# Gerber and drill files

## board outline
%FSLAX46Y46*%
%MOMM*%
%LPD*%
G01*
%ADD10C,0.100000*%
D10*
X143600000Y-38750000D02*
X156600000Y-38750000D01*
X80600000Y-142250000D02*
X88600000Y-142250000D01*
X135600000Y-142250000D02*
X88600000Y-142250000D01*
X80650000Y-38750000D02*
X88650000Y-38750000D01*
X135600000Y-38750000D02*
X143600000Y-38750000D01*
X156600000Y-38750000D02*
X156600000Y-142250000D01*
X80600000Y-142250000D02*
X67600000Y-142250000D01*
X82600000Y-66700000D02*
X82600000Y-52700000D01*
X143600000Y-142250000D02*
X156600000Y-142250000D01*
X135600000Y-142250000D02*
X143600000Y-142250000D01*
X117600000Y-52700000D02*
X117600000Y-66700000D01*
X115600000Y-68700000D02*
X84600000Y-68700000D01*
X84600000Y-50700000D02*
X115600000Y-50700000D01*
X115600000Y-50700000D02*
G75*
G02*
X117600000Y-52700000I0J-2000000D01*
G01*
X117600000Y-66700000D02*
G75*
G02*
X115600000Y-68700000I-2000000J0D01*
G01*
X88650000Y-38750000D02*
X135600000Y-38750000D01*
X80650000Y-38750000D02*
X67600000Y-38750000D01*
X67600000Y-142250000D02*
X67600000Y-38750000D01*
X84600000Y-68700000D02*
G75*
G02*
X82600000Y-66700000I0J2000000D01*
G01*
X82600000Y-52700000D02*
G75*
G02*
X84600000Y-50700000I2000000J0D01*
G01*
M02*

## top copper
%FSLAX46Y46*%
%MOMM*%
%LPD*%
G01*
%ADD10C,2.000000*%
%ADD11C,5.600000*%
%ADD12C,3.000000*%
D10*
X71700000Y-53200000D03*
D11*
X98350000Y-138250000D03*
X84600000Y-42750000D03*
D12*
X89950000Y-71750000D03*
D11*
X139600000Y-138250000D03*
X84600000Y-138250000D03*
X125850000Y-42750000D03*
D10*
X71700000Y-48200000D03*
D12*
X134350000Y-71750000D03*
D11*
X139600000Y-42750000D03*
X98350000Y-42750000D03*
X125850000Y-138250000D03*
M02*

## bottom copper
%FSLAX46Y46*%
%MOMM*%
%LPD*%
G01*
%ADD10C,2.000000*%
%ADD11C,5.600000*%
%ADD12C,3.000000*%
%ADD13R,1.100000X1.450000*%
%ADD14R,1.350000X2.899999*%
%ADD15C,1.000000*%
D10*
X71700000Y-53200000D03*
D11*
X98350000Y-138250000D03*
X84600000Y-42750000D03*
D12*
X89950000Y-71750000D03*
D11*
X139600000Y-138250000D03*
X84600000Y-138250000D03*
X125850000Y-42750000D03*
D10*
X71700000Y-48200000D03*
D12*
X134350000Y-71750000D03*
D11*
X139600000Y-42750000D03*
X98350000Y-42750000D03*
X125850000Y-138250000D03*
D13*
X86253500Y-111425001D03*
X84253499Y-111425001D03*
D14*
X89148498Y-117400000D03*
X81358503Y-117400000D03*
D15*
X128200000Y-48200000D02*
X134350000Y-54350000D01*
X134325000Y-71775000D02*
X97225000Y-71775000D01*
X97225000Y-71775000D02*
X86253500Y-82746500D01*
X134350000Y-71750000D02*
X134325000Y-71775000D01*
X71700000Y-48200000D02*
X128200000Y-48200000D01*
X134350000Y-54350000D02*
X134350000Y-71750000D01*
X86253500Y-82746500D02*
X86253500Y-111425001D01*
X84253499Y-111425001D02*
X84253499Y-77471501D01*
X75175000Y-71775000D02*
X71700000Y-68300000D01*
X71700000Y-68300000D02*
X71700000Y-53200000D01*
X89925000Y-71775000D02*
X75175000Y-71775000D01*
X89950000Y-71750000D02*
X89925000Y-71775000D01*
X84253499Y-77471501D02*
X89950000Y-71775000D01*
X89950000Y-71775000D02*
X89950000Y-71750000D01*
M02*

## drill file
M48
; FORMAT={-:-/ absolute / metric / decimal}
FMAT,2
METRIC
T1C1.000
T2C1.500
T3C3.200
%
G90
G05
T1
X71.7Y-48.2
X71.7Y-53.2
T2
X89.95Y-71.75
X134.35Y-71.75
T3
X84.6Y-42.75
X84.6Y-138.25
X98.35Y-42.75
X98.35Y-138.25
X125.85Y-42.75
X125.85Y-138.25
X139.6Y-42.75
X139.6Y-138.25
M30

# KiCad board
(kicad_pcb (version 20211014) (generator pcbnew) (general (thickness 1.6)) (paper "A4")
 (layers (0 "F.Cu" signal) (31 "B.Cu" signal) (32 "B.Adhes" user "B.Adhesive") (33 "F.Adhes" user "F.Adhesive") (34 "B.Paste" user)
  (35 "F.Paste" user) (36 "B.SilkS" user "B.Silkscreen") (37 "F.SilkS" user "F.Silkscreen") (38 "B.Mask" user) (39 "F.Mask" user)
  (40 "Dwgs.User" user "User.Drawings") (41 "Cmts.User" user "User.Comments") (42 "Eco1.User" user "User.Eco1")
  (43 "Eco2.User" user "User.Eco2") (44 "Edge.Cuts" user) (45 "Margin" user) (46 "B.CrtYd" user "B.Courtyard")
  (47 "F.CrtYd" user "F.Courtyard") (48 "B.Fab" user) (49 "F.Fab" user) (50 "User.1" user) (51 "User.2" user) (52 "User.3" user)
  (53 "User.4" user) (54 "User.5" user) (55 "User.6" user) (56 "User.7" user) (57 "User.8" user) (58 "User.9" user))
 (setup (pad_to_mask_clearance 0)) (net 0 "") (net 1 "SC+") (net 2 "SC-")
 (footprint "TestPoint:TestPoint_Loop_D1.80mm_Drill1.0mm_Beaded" (layer "F.Cu") (at 71.75 53.2)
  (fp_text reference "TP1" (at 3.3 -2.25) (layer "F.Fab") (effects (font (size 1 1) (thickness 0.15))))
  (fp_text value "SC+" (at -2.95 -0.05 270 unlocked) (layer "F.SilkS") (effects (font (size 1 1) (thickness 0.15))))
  (pad "1" thru_hole circle (at -0.05 0) (size 2 2) (drill 1) (layers *.Cu *.Mask) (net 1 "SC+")))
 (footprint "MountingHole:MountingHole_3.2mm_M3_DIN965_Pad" (layer "F.Cu") (at 98.35 138.25)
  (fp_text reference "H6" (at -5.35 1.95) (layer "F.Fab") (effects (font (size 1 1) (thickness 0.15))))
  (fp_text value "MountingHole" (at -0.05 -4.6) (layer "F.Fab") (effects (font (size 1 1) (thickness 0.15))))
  (pad "1" thru_hole circle (at 0 0) (size 5.6 5.6) (drill 3.2) (layers *.Cu *.Mask)))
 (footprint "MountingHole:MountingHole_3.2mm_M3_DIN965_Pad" (layer "F.Cu") (at 84.6 42.75)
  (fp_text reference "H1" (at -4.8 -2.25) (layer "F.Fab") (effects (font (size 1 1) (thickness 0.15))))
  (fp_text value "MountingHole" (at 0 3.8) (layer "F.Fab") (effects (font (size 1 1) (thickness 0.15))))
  (pad "1" thru_hole circle (at 0 0) (size 5.6 5.6) (drill 3.2) (layers *.Cu *.Mask)))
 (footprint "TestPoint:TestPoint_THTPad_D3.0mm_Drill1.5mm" (layer "F.Cu") (at 89.95 71.75)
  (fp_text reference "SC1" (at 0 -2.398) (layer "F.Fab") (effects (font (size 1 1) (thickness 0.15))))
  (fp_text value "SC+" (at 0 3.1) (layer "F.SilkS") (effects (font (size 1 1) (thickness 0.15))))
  (pad "1" thru_hole circle (at 0 0) (size 3 3) (drill 1.5) (layers *.Cu *.Mask) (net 1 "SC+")))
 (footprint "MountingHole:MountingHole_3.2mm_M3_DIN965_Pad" (layer "F.Cu") (at 139.6 138.25)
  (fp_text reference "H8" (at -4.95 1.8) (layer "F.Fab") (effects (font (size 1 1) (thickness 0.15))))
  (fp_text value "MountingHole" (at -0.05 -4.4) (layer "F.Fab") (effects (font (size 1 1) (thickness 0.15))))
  (pad "1" thru_hole circle (at 0 0) (size 5.6 5.6) (drill 3.2) (layers *.Cu *.Mask)))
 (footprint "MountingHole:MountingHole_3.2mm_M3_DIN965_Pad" (layer "F.Cu") (at 84.6 138.25)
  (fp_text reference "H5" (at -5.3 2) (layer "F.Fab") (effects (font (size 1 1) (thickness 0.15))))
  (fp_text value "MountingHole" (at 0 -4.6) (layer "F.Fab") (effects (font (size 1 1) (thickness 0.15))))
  (pad "1" thru_hole circle (at 0 0) (size 5.6 5.6) (drill 3.2) (layers *.Cu *.Mask)))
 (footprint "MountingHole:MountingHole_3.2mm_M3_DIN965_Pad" (layer "F.Cu") (at 125.85 42.75)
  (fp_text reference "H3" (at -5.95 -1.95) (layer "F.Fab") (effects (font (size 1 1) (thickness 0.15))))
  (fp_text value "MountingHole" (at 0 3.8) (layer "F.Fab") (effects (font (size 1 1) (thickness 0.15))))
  (pad "1" thru_hole circle (at 0 0) (size 5.6 5.6) (drill 3.2) (layers *.Cu *.Mask)))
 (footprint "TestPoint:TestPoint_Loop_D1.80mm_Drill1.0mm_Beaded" (layer "F.Cu") (at 71.7 48.3)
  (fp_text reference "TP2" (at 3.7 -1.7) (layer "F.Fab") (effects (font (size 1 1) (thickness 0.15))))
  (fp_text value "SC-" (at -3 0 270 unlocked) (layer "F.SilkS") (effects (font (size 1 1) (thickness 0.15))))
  (pad "1" thru_hole circle (at 0 -0.1) (size 2 2) (drill 1) (layers *.Cu *.Mask) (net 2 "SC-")))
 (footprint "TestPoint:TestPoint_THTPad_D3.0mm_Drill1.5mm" (layer "F.Cu") (at 134.35 71.75)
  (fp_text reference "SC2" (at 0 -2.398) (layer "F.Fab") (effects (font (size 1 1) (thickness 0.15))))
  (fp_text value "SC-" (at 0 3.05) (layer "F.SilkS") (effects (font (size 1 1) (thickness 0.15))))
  (pad "1" thru_hole circle (at 0 0) (size 3 3) (drill 1.5) (layers *.Cu *.Mask) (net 2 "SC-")))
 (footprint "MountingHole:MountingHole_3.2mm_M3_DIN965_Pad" (layer "F.Cu") (at 139.6 42.75)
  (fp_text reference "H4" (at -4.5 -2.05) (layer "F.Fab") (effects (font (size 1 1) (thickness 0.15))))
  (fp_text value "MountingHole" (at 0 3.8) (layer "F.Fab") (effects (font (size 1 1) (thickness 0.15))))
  (pad "1" thru_hole circle (at 0 0) (size 5.6 5.6) (drill 3.2) (layers *.Cu *.Mask)))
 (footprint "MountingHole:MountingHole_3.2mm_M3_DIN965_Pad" (layer "F.Cu") (at 98.35 42.75)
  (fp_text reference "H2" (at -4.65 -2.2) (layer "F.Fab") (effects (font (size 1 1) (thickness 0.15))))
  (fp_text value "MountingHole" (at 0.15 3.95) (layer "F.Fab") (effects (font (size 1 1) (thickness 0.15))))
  (pad "1" thru_hole circle (at 0 0) (size 5.6 5.6) (drill 3.2) (layers *.Cu *.Mask)))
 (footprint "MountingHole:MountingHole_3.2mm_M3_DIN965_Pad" (layer "F.Cu") (at 125.85 138.25)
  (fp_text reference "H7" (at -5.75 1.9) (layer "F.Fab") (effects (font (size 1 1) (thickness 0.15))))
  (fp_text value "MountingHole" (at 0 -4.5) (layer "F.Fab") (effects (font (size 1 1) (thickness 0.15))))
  (pad "1" thru_hole circle (at 0 0) (size 5.6 5.6) (drill 3.2) (layers *.Cu *.Mask)))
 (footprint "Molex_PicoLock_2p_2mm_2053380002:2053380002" (layer "B.Cu") (at 86.2535 111.425001)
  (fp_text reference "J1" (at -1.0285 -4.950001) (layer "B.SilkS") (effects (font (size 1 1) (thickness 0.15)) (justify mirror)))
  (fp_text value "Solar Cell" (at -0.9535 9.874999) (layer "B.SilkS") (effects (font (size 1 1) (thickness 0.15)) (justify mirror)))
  (pad "1" smd rect locked (at 0 0) (size 1.1 1.45) (layers "B.Cu" "B.Paste" "B.Mask") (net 2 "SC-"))
  (pad "2" smd rect locked (at -2.000001 0) (size 1.1 1.45) (layers "B.Cu" "B.Paste" "B.Mask") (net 1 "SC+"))
  (pad "3" smd rect locked (at 2.894998 5.974999) (size 1.35 2.899999) (layers "B.Cu" "B.Paste" "B.Mask"))
  (pad "4" smd rect locked (at -4.894997 5.974999) (size 1.35 2.899999) (layers "B.Cu" "B.Paste" "B.Mask")))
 (gr_line (start 143.6 38.75) (end 156.6 38.75) (layer "Edge.Cuts") (width 0.1))
 (gr_line (start 80.6 142.25) (end 88.6 142.25) (layer "Edge.Cuts") (width 0.1))
 (gr_line (start 135.6 142.25) (end 88.6 142.25) (layer "Edge.Cuts") (width 0.1))
 (gr_line (start 80.65 38.75) (end 88.65 38.75) (layer "Edge.Cuts") (width 0.1))
 (gr_line (start 135.6 38.75) (end 143.6 38.75) (layer "Edge.Cuts") (width 0.1))
 (gr_line (start 156.6 38.75) (end 156.6 142.25) (layer "Edge.Cuts") (width 0.1))
 (gr_line (start 80.6 142.25) (end 67.6 142.25) (layer "Edge.Cuts") (width 0.1))
 (gr_line (start 82.6 66.7) (end 82.6 52.7) (layer "Edge.Cuts") (width 0.1))
 (gr_line (start 143.6 142.25) (end 156.6 142.25) (layer "Edge.Cuts") (width 0.1))
 (gr_line (start 135.6 142.25) (end 143.6 142.25) (layer "Edge.Cuts") (width 0.1))
 (gr_line (start 117.6 52.7) (end 117.6 66.7) (layer "Edge.Cuts") (width 0.1))
 (gr_line (start 115.6 68.7) (end 84.6 68.7) (layer "Edge.Cuts") (width 0.1))
 (gr_line (start 84.6 50.7) (end 115.6 50.7) (layer "Edge.Cuts") (width 0.1))
 (gr_arc (start 115.6 50.7) (mid 117.014214 51.285786) (end 117.6 52.7) (layer "Edge.Cuts") (width 0.1))
 (gr_arc (start 117.6 66.7) (mid 117.014214 68.114214) (end 115.6 68.7) (layer "Edge.Cuts") (width 0.1))
 (gr_line (start 88.65 38.75) (end 135.6 38.75) (layer "Edge.Cuts") (width 0.1))
 (gr_line (start 80.65 38.75) (end 67.6 38.75) (layer "Edge.Cuts") (width 0.1))
 (gr_line (start 67.6 142.25) (end 67.6 38.75) (layer "Edge.Cuts") (width 0.1))
 (gr_arc (start 84.6 68.7) (mid 83.185786 68.114214) (end 82.6 66.7) (layer "Edge.Cuts") (width 0.1))
 (gr_arc (start 82.6 52.7) (mid 83.185786 51.285786) (end 84.6 50.7) (layer "Edge.Cuts") (width 0.1))
 (segment (start 128.2 48.2) (end 134.35 54.35) (width 1) (layer "B.Cu") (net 2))
 (segment (start 134.325 71.775) (end 97.225 71.775) (width 1) (layer "B.Cu") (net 2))
 (segment (start 97.225 71.775) (end 86.2535 82.7465) (width 1) (layer "B.Cu") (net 2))
 (segment (start 134.35 71.75) (end 134.325 71.775) (width 1) (layer "B.Cu") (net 2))
 (segment (start 71.7 48.2) (end 128.2 48.2) (width 1) (layer "B.Cu") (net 2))
 (segment (start 134.35 54.35) (end 134.35 71.75) (width 1) (layer "B.Cu") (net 2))
 (segment (start 86.2535 82.7465) (end 86.2535 111.425001) (width 1) (layer "B.Cu") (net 2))
 (segment (start 84.253499 111.425001) (end 84.253499 77.471501) (width 1) (layer "B.Cu") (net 1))
 (segment (start 75.175 71.775) (end 71.7 68.3) (width 1) (layer "B.Cu") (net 1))
 (segment (start 71.7 68.3) (end 71.7 53.2) (width 1) (layer "B.Cu") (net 1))
 (segment (start 89.925 71.775) (end 75.175 71.775) (width 1) (layer "B.Cu") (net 1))
 (segment (start 89.95 71.75) (end 89.925 71.775) (width 1) (layer "B.Cu") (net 1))
 (segment (start 84.253499 77.471501) (end 89.95 71.775) (width 1) (layer "B.Cu") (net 1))
 (segment (start 89.95 71.775) (end 89.95 71.75) (width 1) (layer "B.Cu") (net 1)))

